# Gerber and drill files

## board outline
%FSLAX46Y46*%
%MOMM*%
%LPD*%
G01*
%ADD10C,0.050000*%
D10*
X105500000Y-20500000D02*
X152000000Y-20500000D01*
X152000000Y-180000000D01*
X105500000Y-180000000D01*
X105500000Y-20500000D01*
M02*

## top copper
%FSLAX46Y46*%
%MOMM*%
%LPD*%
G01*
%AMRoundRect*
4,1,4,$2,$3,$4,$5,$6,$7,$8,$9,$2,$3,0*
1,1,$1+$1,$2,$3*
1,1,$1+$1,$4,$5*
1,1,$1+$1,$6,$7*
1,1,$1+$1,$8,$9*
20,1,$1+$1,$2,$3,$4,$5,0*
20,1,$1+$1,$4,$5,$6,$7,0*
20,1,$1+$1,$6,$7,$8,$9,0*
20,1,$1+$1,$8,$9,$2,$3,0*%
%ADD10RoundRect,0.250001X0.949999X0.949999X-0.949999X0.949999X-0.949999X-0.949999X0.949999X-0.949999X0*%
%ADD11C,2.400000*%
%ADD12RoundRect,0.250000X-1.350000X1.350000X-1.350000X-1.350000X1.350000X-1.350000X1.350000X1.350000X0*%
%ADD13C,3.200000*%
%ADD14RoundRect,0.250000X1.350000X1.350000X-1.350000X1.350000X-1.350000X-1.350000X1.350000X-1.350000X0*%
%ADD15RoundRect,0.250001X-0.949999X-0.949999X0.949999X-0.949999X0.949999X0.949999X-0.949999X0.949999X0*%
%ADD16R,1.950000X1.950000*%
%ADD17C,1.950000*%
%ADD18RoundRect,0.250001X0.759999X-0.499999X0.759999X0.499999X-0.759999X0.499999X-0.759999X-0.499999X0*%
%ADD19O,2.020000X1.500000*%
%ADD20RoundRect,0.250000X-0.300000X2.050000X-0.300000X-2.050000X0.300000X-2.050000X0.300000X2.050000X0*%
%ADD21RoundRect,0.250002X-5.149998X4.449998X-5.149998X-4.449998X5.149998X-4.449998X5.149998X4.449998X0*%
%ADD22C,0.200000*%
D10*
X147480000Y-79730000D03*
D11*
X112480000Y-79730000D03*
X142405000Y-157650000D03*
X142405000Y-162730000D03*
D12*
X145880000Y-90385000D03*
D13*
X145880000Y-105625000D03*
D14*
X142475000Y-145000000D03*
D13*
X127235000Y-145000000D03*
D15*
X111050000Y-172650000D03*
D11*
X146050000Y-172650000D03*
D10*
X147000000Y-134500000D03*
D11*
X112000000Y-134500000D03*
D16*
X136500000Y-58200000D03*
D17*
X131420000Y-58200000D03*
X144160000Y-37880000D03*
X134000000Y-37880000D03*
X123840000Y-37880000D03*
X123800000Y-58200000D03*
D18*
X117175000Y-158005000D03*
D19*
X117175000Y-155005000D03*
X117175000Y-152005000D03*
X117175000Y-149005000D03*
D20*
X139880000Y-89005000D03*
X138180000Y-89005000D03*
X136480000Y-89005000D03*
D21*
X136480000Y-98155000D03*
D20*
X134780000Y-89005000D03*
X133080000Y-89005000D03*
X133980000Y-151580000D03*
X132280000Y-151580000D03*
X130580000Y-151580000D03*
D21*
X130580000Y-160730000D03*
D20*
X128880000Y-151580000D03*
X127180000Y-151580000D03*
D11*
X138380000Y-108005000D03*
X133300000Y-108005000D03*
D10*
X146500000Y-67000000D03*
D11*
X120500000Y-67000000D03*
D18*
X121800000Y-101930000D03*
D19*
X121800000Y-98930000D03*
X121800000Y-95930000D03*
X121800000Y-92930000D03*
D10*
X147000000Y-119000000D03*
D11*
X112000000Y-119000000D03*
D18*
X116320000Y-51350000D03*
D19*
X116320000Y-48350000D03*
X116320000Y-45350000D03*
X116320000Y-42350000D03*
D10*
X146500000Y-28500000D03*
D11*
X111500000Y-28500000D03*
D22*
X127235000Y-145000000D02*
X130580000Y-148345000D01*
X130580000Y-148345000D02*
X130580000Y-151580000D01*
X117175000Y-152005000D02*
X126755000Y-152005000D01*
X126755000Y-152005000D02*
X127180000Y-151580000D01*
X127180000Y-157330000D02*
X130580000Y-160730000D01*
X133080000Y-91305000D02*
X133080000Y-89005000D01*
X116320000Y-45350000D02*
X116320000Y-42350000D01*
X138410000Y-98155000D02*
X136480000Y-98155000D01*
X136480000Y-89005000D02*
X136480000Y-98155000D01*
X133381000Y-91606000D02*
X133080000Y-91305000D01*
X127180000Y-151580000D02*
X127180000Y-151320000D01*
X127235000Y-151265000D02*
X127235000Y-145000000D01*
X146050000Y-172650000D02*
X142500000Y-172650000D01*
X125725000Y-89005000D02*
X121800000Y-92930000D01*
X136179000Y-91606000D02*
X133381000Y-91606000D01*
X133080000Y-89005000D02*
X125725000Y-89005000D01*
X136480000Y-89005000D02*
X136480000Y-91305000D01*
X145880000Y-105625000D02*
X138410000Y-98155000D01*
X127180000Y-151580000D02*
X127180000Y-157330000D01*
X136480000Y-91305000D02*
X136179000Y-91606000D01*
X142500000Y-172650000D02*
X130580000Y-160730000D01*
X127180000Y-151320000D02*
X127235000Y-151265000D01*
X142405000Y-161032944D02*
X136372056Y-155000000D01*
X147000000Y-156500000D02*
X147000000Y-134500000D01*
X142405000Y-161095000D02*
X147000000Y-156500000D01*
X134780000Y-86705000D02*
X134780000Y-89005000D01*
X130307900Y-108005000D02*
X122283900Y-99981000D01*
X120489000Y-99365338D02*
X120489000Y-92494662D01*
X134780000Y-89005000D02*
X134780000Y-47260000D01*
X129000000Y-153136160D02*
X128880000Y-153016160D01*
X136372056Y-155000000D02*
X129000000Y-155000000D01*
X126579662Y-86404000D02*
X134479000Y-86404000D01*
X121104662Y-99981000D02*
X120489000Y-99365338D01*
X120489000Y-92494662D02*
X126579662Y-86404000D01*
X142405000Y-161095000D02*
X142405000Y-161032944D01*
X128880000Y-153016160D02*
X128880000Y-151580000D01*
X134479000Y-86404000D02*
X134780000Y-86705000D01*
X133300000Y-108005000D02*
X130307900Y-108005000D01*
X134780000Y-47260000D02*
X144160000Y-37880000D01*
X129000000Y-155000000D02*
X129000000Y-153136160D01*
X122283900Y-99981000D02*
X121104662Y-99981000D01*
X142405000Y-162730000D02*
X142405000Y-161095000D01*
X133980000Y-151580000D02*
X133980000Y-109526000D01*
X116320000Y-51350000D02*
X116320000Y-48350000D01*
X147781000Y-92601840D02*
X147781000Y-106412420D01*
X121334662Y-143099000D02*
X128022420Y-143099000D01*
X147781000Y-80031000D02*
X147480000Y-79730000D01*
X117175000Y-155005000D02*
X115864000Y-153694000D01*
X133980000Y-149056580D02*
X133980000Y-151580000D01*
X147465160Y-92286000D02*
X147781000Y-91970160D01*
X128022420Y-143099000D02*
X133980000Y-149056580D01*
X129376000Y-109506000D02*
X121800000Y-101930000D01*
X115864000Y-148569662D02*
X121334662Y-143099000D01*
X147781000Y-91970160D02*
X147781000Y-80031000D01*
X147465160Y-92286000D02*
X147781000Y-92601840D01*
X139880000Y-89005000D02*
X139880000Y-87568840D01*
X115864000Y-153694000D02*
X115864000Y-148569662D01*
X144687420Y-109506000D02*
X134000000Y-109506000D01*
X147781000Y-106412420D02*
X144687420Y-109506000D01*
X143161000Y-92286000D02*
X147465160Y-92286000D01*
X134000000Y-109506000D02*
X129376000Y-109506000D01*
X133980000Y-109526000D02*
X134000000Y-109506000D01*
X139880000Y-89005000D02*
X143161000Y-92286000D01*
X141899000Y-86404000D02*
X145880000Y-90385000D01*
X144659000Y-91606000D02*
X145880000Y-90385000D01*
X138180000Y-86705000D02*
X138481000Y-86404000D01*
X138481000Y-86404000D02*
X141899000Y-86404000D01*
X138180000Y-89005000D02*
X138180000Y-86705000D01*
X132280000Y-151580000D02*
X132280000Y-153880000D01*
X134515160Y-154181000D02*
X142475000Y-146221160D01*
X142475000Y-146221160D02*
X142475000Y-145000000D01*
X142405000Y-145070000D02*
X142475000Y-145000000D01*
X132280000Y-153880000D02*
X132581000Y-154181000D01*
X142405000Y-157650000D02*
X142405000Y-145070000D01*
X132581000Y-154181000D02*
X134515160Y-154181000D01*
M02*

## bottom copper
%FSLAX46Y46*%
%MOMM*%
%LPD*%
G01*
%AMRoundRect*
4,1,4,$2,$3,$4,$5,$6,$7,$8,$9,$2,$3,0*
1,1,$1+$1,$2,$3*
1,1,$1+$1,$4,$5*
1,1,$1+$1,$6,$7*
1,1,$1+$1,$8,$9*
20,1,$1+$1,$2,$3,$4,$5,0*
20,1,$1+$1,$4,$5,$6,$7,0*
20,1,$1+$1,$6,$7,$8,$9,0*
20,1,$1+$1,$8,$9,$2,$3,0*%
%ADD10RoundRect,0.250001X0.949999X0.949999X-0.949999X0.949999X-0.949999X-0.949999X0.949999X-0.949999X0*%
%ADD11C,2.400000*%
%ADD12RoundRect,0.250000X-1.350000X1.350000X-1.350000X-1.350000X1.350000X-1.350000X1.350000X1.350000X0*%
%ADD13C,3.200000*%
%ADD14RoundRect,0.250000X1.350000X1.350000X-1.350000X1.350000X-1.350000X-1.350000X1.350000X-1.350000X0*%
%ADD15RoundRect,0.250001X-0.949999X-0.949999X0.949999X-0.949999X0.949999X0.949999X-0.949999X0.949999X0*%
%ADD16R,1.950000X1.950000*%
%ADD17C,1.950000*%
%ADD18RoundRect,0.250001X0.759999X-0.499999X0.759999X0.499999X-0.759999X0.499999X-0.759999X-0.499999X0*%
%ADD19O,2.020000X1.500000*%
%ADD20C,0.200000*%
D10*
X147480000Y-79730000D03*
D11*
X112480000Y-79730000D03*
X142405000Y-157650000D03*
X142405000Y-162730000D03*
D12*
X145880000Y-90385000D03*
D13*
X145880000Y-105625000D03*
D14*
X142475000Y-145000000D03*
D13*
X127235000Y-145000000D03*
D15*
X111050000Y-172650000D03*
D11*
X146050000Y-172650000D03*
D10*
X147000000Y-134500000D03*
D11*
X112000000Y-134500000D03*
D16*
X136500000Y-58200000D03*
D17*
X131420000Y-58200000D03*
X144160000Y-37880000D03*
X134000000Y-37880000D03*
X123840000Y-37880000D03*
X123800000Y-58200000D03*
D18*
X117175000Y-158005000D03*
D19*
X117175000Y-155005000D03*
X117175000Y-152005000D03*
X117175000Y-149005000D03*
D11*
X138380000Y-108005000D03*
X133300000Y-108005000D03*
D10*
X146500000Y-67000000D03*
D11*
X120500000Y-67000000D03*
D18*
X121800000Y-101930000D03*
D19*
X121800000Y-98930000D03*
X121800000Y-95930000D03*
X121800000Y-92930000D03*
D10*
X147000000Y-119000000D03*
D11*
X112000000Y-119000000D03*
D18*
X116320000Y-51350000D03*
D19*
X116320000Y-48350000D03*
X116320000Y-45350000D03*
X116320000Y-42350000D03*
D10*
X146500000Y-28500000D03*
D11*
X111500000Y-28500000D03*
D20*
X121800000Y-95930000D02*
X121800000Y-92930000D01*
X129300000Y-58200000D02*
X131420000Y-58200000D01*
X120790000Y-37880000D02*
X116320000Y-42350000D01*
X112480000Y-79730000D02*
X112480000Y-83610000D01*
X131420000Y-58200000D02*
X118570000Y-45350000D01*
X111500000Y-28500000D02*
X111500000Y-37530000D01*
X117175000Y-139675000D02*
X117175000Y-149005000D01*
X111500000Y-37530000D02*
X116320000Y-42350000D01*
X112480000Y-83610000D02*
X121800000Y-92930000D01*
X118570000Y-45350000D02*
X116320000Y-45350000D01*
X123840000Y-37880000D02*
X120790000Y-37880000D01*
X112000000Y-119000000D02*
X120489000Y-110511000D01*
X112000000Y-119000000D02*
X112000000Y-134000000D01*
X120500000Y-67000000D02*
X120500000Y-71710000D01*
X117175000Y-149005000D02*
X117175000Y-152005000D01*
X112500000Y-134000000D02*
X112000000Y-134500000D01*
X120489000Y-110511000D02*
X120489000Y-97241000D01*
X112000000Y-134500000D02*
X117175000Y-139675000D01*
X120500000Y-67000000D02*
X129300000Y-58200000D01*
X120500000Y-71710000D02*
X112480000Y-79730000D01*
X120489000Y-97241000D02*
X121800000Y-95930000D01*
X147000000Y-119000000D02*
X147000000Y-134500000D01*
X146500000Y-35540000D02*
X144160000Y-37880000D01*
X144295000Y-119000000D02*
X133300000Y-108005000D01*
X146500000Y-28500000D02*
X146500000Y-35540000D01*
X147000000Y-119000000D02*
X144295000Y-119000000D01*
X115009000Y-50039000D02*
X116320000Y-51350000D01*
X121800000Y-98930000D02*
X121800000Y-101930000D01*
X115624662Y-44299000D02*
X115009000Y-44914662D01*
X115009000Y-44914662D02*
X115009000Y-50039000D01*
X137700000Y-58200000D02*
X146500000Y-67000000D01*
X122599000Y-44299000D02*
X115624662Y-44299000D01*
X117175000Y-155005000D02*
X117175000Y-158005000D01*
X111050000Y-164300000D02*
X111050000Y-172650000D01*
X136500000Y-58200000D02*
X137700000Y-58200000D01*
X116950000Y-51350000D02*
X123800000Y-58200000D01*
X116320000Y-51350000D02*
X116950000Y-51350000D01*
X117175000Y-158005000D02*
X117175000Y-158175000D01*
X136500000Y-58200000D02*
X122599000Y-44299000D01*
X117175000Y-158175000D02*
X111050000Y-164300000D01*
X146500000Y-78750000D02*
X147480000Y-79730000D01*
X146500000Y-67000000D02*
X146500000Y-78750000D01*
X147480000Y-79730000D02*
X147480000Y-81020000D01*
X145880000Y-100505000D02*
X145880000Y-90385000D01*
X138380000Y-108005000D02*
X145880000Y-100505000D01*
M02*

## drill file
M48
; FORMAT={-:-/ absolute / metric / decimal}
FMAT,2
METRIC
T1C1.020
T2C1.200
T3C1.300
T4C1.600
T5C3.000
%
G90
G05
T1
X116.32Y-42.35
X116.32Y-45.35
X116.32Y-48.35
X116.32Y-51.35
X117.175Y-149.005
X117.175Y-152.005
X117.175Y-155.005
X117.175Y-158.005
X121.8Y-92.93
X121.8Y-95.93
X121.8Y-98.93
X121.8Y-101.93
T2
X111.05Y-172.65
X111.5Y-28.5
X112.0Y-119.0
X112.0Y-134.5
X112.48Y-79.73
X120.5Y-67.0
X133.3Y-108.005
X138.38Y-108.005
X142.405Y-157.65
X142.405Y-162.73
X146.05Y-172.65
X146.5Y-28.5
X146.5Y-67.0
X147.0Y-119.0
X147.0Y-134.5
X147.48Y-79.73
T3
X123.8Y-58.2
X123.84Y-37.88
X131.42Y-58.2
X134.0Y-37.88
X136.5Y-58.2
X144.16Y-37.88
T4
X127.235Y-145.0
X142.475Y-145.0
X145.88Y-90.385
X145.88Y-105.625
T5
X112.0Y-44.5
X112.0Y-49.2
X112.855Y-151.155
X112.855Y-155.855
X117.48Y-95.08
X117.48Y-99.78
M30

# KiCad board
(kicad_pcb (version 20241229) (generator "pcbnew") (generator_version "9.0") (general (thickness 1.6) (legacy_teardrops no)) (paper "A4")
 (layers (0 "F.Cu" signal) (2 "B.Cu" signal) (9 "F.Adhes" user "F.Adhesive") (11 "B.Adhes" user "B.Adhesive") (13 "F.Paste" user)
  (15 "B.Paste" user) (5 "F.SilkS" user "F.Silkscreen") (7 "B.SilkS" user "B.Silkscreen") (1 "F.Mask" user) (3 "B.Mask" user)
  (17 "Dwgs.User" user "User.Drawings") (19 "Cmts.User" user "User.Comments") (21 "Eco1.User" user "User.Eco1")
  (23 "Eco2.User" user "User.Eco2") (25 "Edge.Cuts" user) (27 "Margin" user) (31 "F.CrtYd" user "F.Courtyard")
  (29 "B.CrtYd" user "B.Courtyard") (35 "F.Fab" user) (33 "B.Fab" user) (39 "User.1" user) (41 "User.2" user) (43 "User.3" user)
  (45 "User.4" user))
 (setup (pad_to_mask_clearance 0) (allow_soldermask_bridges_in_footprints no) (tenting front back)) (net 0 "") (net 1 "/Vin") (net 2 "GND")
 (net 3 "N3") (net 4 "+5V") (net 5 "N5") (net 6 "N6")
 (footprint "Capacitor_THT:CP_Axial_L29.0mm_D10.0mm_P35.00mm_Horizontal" (layer "F.Cu") (at 147.48 79.73 180)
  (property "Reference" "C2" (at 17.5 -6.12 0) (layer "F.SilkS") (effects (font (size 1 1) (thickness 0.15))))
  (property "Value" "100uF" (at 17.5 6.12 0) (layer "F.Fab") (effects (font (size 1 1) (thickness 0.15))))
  (pad "1" thru_hole roundrect (at 0 0 180) (size 2.4 2.4) (drill 1.2) (layers "*.Cu" "*.Mask") (remove_unused_layers no)
   (roundrect_rratio 0.104167) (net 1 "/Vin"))
  (pad "2" thru_hole circle (at 35 0 180) (size 2.4 2.4) (drill 1.2) (layers "*.Cu" "*.Mask") (remove_unused_layers no) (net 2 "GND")))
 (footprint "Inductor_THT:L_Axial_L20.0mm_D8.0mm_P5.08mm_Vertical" (layer "F.Cu") (at 142.405 157.65 -90)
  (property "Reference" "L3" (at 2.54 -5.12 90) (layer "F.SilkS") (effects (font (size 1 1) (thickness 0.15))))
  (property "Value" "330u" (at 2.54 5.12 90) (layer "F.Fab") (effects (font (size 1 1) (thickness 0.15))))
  (pad "1" thru_hole circle (at 0 0 270) (size 2.4 2.4) (drill 1.2) (layers "*.Cu" "*.Mask") (remove_unused_layers no) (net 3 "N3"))
  (pad "2" thru_hole circle (at 5.08 0 270) (size 2.4 2.4) (drill 1.2) (layers "*.Cu" "*.Mask") (remove_unused_layers no) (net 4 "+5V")))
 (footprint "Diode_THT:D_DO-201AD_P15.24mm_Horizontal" (layer "F.Cu") (at 145.88 90.385 -90)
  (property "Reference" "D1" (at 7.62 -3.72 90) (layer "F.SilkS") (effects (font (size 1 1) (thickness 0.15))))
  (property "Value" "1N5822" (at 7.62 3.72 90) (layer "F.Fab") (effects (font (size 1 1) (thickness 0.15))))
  (pad "1" thru_hole roundrect (at 0 0 270) (size 3.2 3.2) (drill 1.6) (layers "*.Cu" "*.Mask") (remove_unused_layers no)
   (roundrect_rratio 0.078125) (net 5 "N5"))
  (pad "2" thru_hole circle (at 15.24 0 270) (size 3.2 3.2) (drill 1.6) (layers "*.Cu" "*.Mask") (remove_unused_layers no) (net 2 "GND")))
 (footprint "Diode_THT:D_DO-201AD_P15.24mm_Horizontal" (layer "F.Cu") (at 142.475 145 180)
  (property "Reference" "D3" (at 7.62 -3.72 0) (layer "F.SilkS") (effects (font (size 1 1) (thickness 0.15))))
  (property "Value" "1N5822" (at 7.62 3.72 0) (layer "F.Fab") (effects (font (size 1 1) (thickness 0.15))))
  (pad "1" thru_hole roundrect (at 0 0 180) (size 3.2 3.2) (drill 1.6) (layers "*.Cu" "*.Mask") (remove_unused_layers no)
   (roundrect_rratio 0.078125) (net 3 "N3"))
  (pad "2" thru_hole circle (at 15.24 0 180) (size 3.2 3.2) (drill 1.6) (layers "*.Cu" "*.Mask") (remove_unused_layers no) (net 2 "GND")))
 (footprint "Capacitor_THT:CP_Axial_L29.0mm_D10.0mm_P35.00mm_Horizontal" (layer "F.Cu") (at 111.05 172.65)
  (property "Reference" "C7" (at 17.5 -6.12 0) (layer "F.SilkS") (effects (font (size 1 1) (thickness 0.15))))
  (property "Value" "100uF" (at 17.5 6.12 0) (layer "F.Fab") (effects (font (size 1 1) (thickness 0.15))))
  (pad "1" thru_hole roundrect (at 0 0) (size 2.4 2.4) (drill 1.2) (layers "*.Cu" "*.Mask") (remove_unused_layers no)
   (roundrect_rratio 0.104167) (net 1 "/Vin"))
  (pad "2" thru_hole circle (at 35 0) (size 2.4 2.4) (drill 1.2) (layers "*.Cu" "*.Mask") (remove_unused_layers no) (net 2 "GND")))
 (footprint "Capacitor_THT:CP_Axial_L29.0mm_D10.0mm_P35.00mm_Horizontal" (layer "F.Cu") (at 147 134.5 180)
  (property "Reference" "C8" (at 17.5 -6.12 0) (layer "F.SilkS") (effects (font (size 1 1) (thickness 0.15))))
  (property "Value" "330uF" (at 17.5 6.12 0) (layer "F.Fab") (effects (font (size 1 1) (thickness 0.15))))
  (pad "1" thru_hole roundrect (at 0 0 180) (size 2.4 2.4) (drill 1.2) (layers "*.Cu" "*.Mask") (remove_unused_layers no)
   (roundrect_rratio 0.104167) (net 4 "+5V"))
  (pad "2" thru_hole circle (at 35 0 180) (size 2.4 2.4) (drill 1.2) (layers "*.Cu" "*.Mask") (remove_unused_layers no) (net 2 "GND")))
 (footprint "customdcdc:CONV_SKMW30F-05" (layer "F.Cu") (at 134 48 180)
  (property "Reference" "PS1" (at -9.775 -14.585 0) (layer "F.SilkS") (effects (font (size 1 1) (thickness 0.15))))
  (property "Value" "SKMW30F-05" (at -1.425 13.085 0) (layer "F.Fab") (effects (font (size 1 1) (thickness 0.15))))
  (pad "1" thru_hole rect (at -2.5 -10.2 180) (size 1.95 1.95) (drill 1.3) (layers "*.Cu" "*.Mask") (remove_unused_layers no) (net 1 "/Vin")
   (solder_mask_margin 0.102))
  (pad "2" thru_hole circle (at 2.58 -10.2 180) (size 1.95 1.95) (drill 1.3) (layers "*.Cu" "*.Mask") (remove_unused_layers no)
   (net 2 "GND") (solder_mask_margin 0.102))
  (pad "3" thru_hole circle (at -10.16 10.12 180) (size 1.95 1.95) (drill 1.3) (layers "*.Cu" "*.Mask") (remove_unused_layers no)
   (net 4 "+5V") (solder_mask_margin 0.102))
  (pad "4" thru_hole circle (at 0 10.12 180) (size 1.95 1.95) (drill 1.3) (layers "*.Cu" "*.Mask") (remove_unused_layers no) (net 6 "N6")
   (solder_mask_margin 0.102))
  (pad "5" thru_hole circle (at 10.16 10.12 180) (size 1.95 1.95) (drill 1.3) (layers "*.Cu" "*.Mask") (remove_unused_layers no)
   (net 2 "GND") (solder_mask_margin 0.102))
  (pad "6" thru_hole circle (at 10.2 -10.2 180) (size 1.95 1.95) (drill 1.3) (layers "*.Cu" "*.Mask") (remove_unused_layers no)
   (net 1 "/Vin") (solder_mask_margin 0.102)))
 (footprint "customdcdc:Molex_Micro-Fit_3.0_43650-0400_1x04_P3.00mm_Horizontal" (layer "F.Cu") (at 117.175 158.005 90)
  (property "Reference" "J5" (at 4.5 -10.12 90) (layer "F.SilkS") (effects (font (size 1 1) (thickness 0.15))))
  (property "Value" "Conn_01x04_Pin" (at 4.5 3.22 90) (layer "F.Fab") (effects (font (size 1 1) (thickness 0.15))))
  (pad "" np_thru_hole circle (at 2.15 -4.32 90) (size 3 3) (drill 3) (layers "*.Cu" "*.Mask"))
  (pad "" np_thru_hole circle (at 6.85 -4.32 90) (size 3 3) (drill 3) (layers "*.Cu" "*.Mask"))
  (pad "1" thru_hole roundrect (at 0 0 90) (size 1.5 2.02) (drill 1.02) (layers "*.Cu" "*.Mask") (remove_unused_layers no)
   (roundrect_rratio 0.166667) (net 1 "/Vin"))
  (pad "2" thru_hole oval (at 3 0 90) (size 1.5 2.02) (drill 1.02) (layers "*.Cu" "*.Mask") (remove_unused_layers no) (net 1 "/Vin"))
  (pad "3" thru_hole oval (at 6 0 90) (size 1.5 2.02) (drill 1.02) (layers "*.Cu" "*.Mask") (remove_unused_layers no) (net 2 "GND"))
  (pad "4" thru_hole oval (at 9 0 90) (size 1.5 2.02) (drill 1.02) (layers "*.Cu" "*.Mask") (remove_unused_layers no) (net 2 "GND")))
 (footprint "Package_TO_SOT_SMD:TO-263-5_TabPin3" (layer "F.Cu") (at 136.48 96.655 -90)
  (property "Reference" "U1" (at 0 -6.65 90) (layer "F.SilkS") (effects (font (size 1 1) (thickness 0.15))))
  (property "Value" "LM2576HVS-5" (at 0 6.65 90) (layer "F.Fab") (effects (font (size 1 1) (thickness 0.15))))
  (pad "" smd roundrect (at -0.925 -2.775 270) (size 4.55 5.25) (layers "F.Paste") (roundrect_rratio 0.054945))
  (pad "" smd roundrect (at -0.925 2.775 270) (size 4.55 5.25) (layers "F.Paste") (roundrect_rratio 0.054945))
  (pad "" smd roundrect (at 3.925 -2.775 270) (size 4.55 5.25) (layers "F.Paste") (roundrect_rratio 0.054945))
  (pad "" smd roundrect (at 3.925 2.775 270) (size 4.55 5.25) (layers "F.Paste") (roundrect_rratio 0.054945))
  (pad "1" smd roundrect (at -7.65 -3.4 270) (size 4.6 1.1) (layers "F.Cu" "F.Mask" "F.Paste") (roundrect_rratio 0.227273) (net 1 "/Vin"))
  (pad "2" smd roundrect (at -7.65 -1.7 270) (size 4.6 1.1) (layers "F.Cu" "F.Mask" "F.Paste") (roundrect_rratio 0.227273) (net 5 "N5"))
  (pad "3" smd roundrect (at -7.65 0 270) (size 4.6 1.1) (layers "F.Cu" "F.Mask" "F.Paste") (roundrect_rratio 0.227273) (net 2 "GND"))
  (pad "3" smd roundrect (at 1.5 0 270) (size 9.4 10.8) (layers "F.Cu" "F.Mask") (roundrect_rratio 0.026596) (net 2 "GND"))
  (pad "4" smd roundrect (at -7.65 1.7 270) (size 4.6 1.1) (layers "F.Cu" "F.Mask" "F.Paste") (roundrect_rratio 0.227273) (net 4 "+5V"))
  (pad "5" smd roundrect (at -7.65 3.4 270) (size 4.6 1.1) (layers "F.Cu" "F.Mask" "F.Paste") (roundrect_rratio 0.227273) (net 2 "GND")))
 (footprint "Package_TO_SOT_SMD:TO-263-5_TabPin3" (layer "F.Cu") (at 130.58 159.23 -90)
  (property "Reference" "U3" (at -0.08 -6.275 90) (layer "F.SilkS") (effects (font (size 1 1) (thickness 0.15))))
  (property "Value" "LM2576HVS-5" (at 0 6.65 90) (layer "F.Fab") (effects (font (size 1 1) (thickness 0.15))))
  (pad "" smd roundrect (at -0.925 -2.775 270) (size 4.55 5.25) (layers "F.Paste") (roundrect_rratio 0.054945))
  (pad "" smd roundrect (at -0.925 2.775 270) (size 4.55 5.25) (layers "F.Paste") (roundrect_rratio 0.054945))
  (pad "" smd roundrect (at 3.925 -2.775 270) (size 4.55 5.25) (layers "F.Paste") (roundrect_rratio 0.054945))
  (pad "" smd roundrect (at 3.925 2.775 270) (size 4.55 5.25) (layers "F.Paste") (roundrect_rratio 0.054945))
  (pad "1" smd roundrect (at -7.65 -3.4 270) (size 4.6 1.1) (layers "F.Cu" "F.Mask" "F.Paste") (roundrect_rratio 0.227273) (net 1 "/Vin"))
  (pad "2" smd roundrect (at -7.65 -1.7 270) (size 4.6 1.1) (layers "F.Cu" "F.Mask" "F.Paste") (roundrect_rratio 0.227273) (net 3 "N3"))
  (pad "3" smd roundrect (at -7.65 0 270) (size 4.6 1.1) (layers "F.Cu" "F.Mask" "F.Paste") (roundrect_rratio 0.227273) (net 2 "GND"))
  (pad "3" smd roundrect (at 1.5 0 270) (size 9.4 10.8) (layers "F.Cu" "F.Mask") (roundrect_rratio 0.026596) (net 2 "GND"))
  (pad "4" smd roundrect (at -7.65 1.7 270) (size 4.6 1.1) (layers "F.Cu" "F.Mask" "F.Paste") (roundrect_rratio 0.227273) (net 4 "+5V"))
  (pad "5" smd roundrect (at -7.65 3.4 270) (size 4.6 1.1) (layers "F.Cu" "F.Mask" "F.Paste") (roundrect_rratio 0.227273) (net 2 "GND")))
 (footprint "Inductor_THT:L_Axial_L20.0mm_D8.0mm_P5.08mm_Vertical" (layer "F.Cu") (at 138.38 108.005 180)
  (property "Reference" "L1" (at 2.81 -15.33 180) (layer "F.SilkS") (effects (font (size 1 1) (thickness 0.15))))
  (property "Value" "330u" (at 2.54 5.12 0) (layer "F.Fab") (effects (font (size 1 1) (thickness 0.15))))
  (pad "1" thru_hole circle (at 0 0 180) (size 2.4 2.4) (drill 1.2) (layers "*.Cu" "*.Mask") (remove_unused_layers no) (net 5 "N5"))
  (pad "2" thru_hole circle (at 5.08 0 180) (size 2.4 2.4) (drill 1.2) (layers "*.Cu" "*.Mask") (remove_unused_layers no) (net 4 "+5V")))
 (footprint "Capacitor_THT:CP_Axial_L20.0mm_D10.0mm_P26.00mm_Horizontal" (layer "F.Cu") (at 146.5 67 180)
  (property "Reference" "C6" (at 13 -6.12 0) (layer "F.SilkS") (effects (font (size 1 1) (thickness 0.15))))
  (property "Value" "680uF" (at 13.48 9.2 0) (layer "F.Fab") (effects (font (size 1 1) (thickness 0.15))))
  (pad "1" thru_hole roundrect (at 0 0 180) (size 2.4 2.4) (drill 1.2) (layers "*.Cu" "*.Mask") (remove_unused_layers no)
   (roundrect_rratio 0.104167) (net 1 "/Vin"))
  (pad "2" thru_hole circle (at 26 0 180) (size 2.4 2.4) (drill 1.2) (layers "*.Cu" "*.Mask") (remove_unused_layers no) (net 2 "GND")))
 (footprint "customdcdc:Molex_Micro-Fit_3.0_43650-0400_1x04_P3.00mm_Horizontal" (layer "F.Cu") (at 121.8 101.93 90)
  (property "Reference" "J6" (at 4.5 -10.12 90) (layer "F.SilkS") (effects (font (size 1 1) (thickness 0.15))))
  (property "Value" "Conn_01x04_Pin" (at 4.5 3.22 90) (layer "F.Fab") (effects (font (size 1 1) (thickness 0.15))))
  (pad "" np_thru_hole circle (at 2.15 -4.32 90) (size 3 3) (drill 3) (layers "*.Cu" "*.Mask"))
  (pad "" np_thru_hole circle (at 6.85 -4.32 90) (size 3 3) (drill 3) (layers "*.Cu" "*.Mask"))
  (pad "1" thru_hole roundrect (at 0 0 90) (size 1.5 2.02) (drill 1.02) (layers "*.Cu" "*.Mask") (remove_unused_layers no)
   (roundrect_rratio 0.166667) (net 1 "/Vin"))
  (pad "2" thru_hole oval (at 3 0 90) (size 1.5 2.02) (drill 1.02) (layers "*.Cu" "*.Mask") (remove_unused_layers no) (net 1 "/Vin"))
  (pad "3" thru_hole oval (at 6 0 90) (size 1.5 2.02) (drill 1.02) (layers "*.Cu" "*.Mask") (remove_unused_layers no) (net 2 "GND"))
  (pad "4" thru_hole oval (at 9 0 90) (size 1.5 2.02) (drill 1.02) (layers "*.Cu" "*.Mask") (remove_unused_layers no) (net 2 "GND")))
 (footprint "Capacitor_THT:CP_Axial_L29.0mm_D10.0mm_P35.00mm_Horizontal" (layer "F.Cu") (at 147 119 180)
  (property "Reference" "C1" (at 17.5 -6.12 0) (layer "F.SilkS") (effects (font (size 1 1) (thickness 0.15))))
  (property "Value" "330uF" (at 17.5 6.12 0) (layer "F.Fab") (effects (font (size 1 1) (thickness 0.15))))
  (pad "1" thru_hole roundrect (at 0 0 180) (size 2.4 2.4) (drill 1.2) (layers "*.Cu" "*.Mask") (remove_unused_layers no)
   (roundrect_rratio 0.104167) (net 4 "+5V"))
  (pad "2" thru_hole circle (at 35 0 180) (size 2.4 2.4) (drill 1.2) (layers "*.Cu" "*.Mask") (remove_unused_layers no) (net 2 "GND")))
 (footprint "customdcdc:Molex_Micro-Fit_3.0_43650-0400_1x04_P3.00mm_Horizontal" (layer "F.Cu") (at 116.32 51.35 90)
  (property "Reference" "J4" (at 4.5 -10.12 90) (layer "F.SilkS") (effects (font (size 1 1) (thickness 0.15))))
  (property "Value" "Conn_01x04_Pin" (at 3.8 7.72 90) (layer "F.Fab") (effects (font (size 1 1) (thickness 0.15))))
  (pad "" np_thru_hole circle (at 2.15 -4.32 90) (size 3 3) (drill 3) (layers "*.Cu" "*.Mask"))
  (pad "" np_thru_hole circle (at 6.85 -4.32 90) (size 3 3) (drill 3) (layers "*.Cu" "*.Mask"))
  (pad "1" thru_hole roundrect (at 0 0 90) (size 1.5 2.02) (drill 1.02) (layers "*.Cu" "*.Mask") (remove_unused_layers no)
   (roundrect_rratio 0.166667) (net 1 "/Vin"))
  (pad "2" thru_hole oval (at 3 0 90) (size 1.5 2.02) (drill 1.02) (layers "*.Cu" "*.Mask") (remove_unused_layers no) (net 1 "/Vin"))
  (pad "3" thru_hole oval (at 6 0 90) (size 1.5 2.02) (drill 1.02) (layers "*.Cu" "*.Mask") (remove_unused_layers no) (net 2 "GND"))
  (pad "4" thru_hole oval (at 9 0 90) (size 1.5 2.02) (drill 1.02) (layers "*.Cu" "*.Mask") (remove_unused_layers no) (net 2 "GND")))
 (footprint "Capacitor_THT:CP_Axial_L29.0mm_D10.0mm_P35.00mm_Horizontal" (layer "F.Cu") (at 146.5 28.5 180)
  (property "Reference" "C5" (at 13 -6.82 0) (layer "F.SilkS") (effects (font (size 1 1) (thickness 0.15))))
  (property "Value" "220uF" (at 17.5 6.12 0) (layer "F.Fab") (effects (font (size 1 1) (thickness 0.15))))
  (pad "1" thru_hole roundrect (at 0 0 180) (size 2.4 2.4) (drill 1.2) (layers "*.Cu" "*.Mask") (remove_unused_layers no)
   (roundrect_rratio 0.104167) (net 4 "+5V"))
  (pad "2" thru_hole circle (at 35 0 180) (size 2.4 2.4) (drill 1.2) (layers "*.Cu" "*.Mask") (remove_unused_layers no) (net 2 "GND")))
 (gr_rect (start 105.5 20.5) (end 152 180) (stroke (width 0.05) (type default)) (fill no) (layer "Edge.Cuts"))
 (segment (start 127.235 145) (end 130.58 148.345) (width 0.2) (layer "F.Cu") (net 2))
 (segment (start 130.58 148.345) (end 130.58 151.58) (width 0.2) (layer "F.Cu") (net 2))
 (segment (start 117.175 152.005) (end 126.755 152.005) (width 0.2) (layer "F.Cu") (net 2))
 (segment (start 126.755 152.005) (end 127.18 151.58) (width 0.2) (layer "F.Cu") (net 2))
 (segment (start 127.18 157.33) (end 130.58 160.73) (width 0.2) (layer "F.Cu") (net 2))
 (segment (start 133.08 91.305) (end 133.08 89.005) (width 0.2) (layer "F.Cu") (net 2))
 (segment (start 116.32 45.35) (end 116.32 42.35) (width 0.2) (layer "F.Cu") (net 2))
 (segment (start 138.41 98.155) (end 136.48 98.155) (width 0.2) (layer "F.Cu") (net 2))
 (segment (start 136.48 89.005) (end 136.48 98.155) (width 0.2) (layer "F.Cu") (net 2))
 (segment (start 133.381 91.606) (end 133.08 91.305) (width 0.2) (layer "F.Cu") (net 2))
 (segment (start 127.18 151.58) (end 127.18 151.32) (width 0.2) (layer "F.Cu") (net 2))
 (segment (start 127.235 151.265) (end 127.235 145) (width 0.2) (layer "F.Cu") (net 2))
 (segment (start 146.05 172.65) (end 142.5 172.65) (width 0.2) (layer "F.Cu") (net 2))
 (segment (start 125.725 89.005) (end 121.8 92.93) (width 0.2) (layer "F.Cu") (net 2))
 (segment (start 136.179 91.606) (end 133.381 91.606) (width 0.2) (layer "F.Cu") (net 2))
 (segment (start 133.08 89.005) (end 125.725 89.005) (width 0.2) (layer "F.Cu") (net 2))
 (segment (start 136.48 89.005) (end 136.48 91.305) (width 0.2) (layer "F.Cu") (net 2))
 (segment (start 145.88 105.625) (end 138.41 98.155) (width 0.2) (layer "F.Cu") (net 2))
 (segment (start 127.18 151.58) (end 127.18 157.33) (width 0.2) (layer "F.Cu") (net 2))
 (segment (start 136.48 91.305) (end 136.179 91.606) (width 0.2) (layer "F.Cu") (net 2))
 (segment (start 142.5 172.65) (end 130.58 160.73) (width 0.2) (layer "F.Cu") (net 2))
 (segment (start 127.18 151.32) (end 127.235 151.265) (width 0.2) (layer "F.Cu") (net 2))
 (segment (start 121.8 95.93) (end 121.8 92.93) (width 0.2) (layer "B.Cu") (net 2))
 (segment (start 129.3 58.2) (end 131.42 58.2) (width 0.2) (layer "B.Cu") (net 2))
 (segment (start 120.79 37.88) (end 116.32 42.35) (width 0.2) (layer "B.Cu") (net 2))
 (segment (start 112.48 79.73) (end 112.48 83.61) (width 0.2) (layer "B.Cu") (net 2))
 (segment (start 131.42 58.2) (end 118.57 45.35) (width 0.2) (layer "B.Cu") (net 2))
 (segment (start 111.5 28.5) (end 111.5 37.53) (width 0.2) (layer "B.Cu") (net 2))
 (segment (start 117.175 139.675) (end 117.175 149.005) (width 0.2) (layer "B.Cu") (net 2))
 (segment (start 111.5 37.53) (end 116.32 42.35) (width 0.2) (layer "B.Cu") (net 2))
 (segment (start 112.48 83.61) (end 121.8 92.93) (width 0.2) (layer "B.Cu") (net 2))
 (segment (start 118.57 45.35) (end 116.32 45.35) (width 0.2) (layer "B.Cu") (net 2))
 (segment (start 123.84 37.88) (end 120.79 37.88) (width 0.2) (layer "B.Cu") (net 2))
 (segment (start 112 119) (end 120.489 110.511) (width 0.2) (layer "B.Cu") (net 2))
 (segment (start 112 119) (end 112 134) (width 0.2) (layer "B.Cu") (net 2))
 (segment (start 120.5 67) (end 120.5 71.71) (width 0.2) (layer "B.Cu") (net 2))
 (segment (start 117.175 149.005) (end 117.175 152.005) (width 0.2) (layer "B.Cu") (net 2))
 (segment (start 112.5 134) (end 112 134.5) (width 0.2) (layer "B.Cu") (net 2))
 (segment (start 120.489 110.511) (end 120.489 97.241) (width 0.2) (layer "B.Cu") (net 2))
 (segment (start 112 134.5) (end 117.175 139.675) (width 0.2) (layer "B.Cu") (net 2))
 (segment (start 120.5 67) (end 129.3 58.2) (width 0.2) (layer "B.Cu") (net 2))
 (segment (start 120.5 71.71) (end 112.48 79.73) (width 0.2) (layer "B.Cu") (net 2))
 (segment (start 120.489 97.241) (end 121.8 95.93) (width 0.2) (layer "B.Cu") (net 2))
 (segment (start 142.405 161.032944) (end 136.372056 155) (width 0.2) (layer "F.Cu") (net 4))
 (segment (start 147 156.5) (end 147 134.5) (width 0.2) (layer "F.Cu") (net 4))
 (segment (start 142.405 161.095) (end 147 156.5) (width 0.2) (layer "F.Cu") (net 4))
 (segment (start 134.78 86.705) (end 134.78 89.005) (width 0.2) (layer "F.Cu") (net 4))
 (segment (start 130.3079 108.005) (end 122.2839 99.981) (width 0.2) (layer "F.Cu") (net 4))
 (segment (start 120.489 99.365338) (end 120.489 92.494662) (width 0.2) (layer "F.Cu") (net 4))
 (segment (start 134.78 89.005) (end 134.78 47.26) (width 0.2) (layer "F.Cu") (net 4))
 (segment (start 129 153.13616) (end 128.88 153.01616) (width 0.2) (layer "F.Cu") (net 4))
 (segment (start 136.372056 155) (end 129 155) (width 0.2) (layer "F.Cu") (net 4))
 (segment (start 126.579662 86.404) (end 134.479 86.404) (width 0.2) (layer "F.Cu") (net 4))
 (segment (start 121.104662 99.981) (end 120.489 99.365338) (width 0.2) (layer "F.Cu") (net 4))
 (segment (start 120.489 92.494662) (end 126.579662 86.404) (width 0.2) (layer "F.Cu") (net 4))
 (segment (start 142.405 161.095) (end 142.405 161.032944) (width 0.2) (layer "F.Cu") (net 4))
 (segment (start 128.88 153.01616) (end 128.88 151.58) (width 0.2) (layer "F.Cu") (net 4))
 (segment (start 134.479 86.404) (end 134.78 86.705) (width 0.2) (layer "F.Cu") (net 4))
 (segment (start 133.3 108.005) (end 130.3079 108.005) (width 0.2) (layer "F.Cu") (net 4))
 (segment (start 134.78 47.26) (end 144.16 37.88) (width 0.2) (layer "F.Cu") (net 4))
 (segment (start 129 155) (end 129 153.13616) (width 0.2) (layer "F.Cu") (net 4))
 (segment (start 122.2839 99.981) (end 121.104662 99.981) (width 0.2) (layer "F.Cu") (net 4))
 (segment (start 142.405 162.73) (end 142.405 161.095) (width 0.2) (layer "F.Cu") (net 4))
 (segment (start 147 119) (end 147 134.5) (width 0.2) (layer "B.Cu") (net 4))
 (segment (start 146.5 35.54) (end 144.16 37.88) (width 0.2) (layer "B.Cu") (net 4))
 (segment (start 144.295 119) (end 133.3 108.005) (width 0.2) (layer "B.Cu") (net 4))
 (segment (start 146.5 28.5) (end 146.5 35.54) (width 0.2) (layer "B.Cu") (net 4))
 (segment (start 147 119) (end 144.295 119) (width 0.2) (layer "B.Cu") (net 4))
 (segment (start 133.98 151.58) (end 133.98 109.526) (width 0.2) (layer "F.Cu") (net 1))
 (segment (start 116.32 51.35) (end 116.32 48.35) (width 0.2) (layer "F.Cu") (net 1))
 (segment (start 147.781 92.60184) (end 147.781 106.41242) (width 0.2) (layer "F.Cu") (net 1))
 (segment (start 121.334662 143.099) (end 128.02242 143.099) (width 0.2) (layer "F.Cu") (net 1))
 (segment (start 147.781 80.031) (end 147.48 79.73) (width 0.2) (layer "F.Cu") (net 1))
 (segment (start 117.175 155.005) (end 115.864 153.694) (width 0.2) (layer "F.Cu") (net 1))
 (segment (start 133.98 149.05658) (end 133.98 151.58) (width 0.2) (layer "F.Cu") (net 1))
 (segment (start 147.46516 92.286) (end 147.781 91.97016) (width 0.2) (layer "F.Cu") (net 1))
 (segment (start 128.02242 143.099) (end 133.98 149.05658) (width 0.2) (layer "F.Cu") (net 1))
 (segment (start 129.376 109.506) (end 121.8 101.93) (width 0.2) (layer "F.Cu") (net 1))
 (segment (start 115.864 148.569662) (end 121.334662 143.099) (width 0.2) (layer "F.Cu") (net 1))
 (segment (start 147.781 91.97016) (end 147.781 80.031) (width 0.2) (layer "F.Cu") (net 1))
 (segment (start 147.46516 92.286) (end 147.781 92.60184) (width 0.2) (layer "F.Cu") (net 1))
 (segment (start 139.88 89.005) (end 139.88 87.56884) (width 0.2) (layer "F.Cu") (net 1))
 (segment (start 115.864 153.694) (end 115.864 148.569662) (width 0.2) (layer "F.Cu") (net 1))
 (segment (start 144.68742 109.506) (end 134 109.506) (width 0.2) (layer "F.Cu") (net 1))
 (segment (start 147.781 106.41242) (end 144.68742 109.506) (width 0.2) (layer "F.Cu") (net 1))
 (segment (start 143.161 92.286) (end 147.46516 92.286) (width 0.2) (layer "F.Cu") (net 1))
 (segment (start 134 109.506) (end 129.376 109.506) (width 0.2) (layer "F.Cu") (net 1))
 (segment (start 133.98 109.526) (end 134 109.506) (width 0.2) (layer "F.Cu") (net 1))
 (segment (start 139.88 89.005) (end 143.161 92.286) (width 0.2) (layer "F.Cu") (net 1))
 (segment (start 115.009 50.039) (end 116.32 51.35) (width 0.2) (layer "B.Cu") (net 1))
 (segment (start 121.8 98.93) (end 121.8 101.93) (width 0.2) (layer "B.Cu") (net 1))
 (segment (start 115.624662 44.299) (end 115.009 44.914662) (width 0.2) (layer "B.Cu") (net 1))
 (segment (start 115.009 44.914662) (end 115.009 50.039) (width 0.2) (layer "B.Cu") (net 1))
 (segment (start 137.7 58.2) (end 146.5 67) (width 0.2) (layer "B.Cu") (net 1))
 (segment (start 122.599 44.299) (end 115.624662 44.299) (width 0.2) (layer "B.Cu") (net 1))
 (segment (start 117.175 155.005) (end 117.175 158.005) (width 0.2) (layer "B.Cu") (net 1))
 (segment (start 111.05 164.3) (end 111.05 172.65) (width 0.2) (layer "B.Cu") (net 1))
 (segment (start 136.5 58.2) (end 137.7 58.2) (width 0.2) (layer "B.Cu") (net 1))
 (segment (start 116.95 51.35) (end 123.8 58.2) (width 0.2) (layer "B.Cu") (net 1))
 (segment (start 116.32 51.35) (end 116.95 51.35) (width 0.2) (layer "B.Cu") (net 1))
 (segment (start 117.175 158.005) (end 117.175 158.175) (width 0.2) (layer "B.Cu") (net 1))
 (segment (start 136.5 58.2) (end 122.599 44.299) (width 0.2) (layer "B.Cu") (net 1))
 (segment (start 117.175 158.175) (end 111.05 164.3) (width 0.2) (layer "B.Cu") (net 1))
 (segment (start 146.5 78.75) (end 147.48 79.73) (width 0.2) (layer "B.Cu") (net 1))
 (segment (start 146.5 67) (end 146.5 78.75) (width 0.2) (layer "B.Cu") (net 1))
 (segment (start 147.48 79.73) (end 147.48 81.02) (width 0.2) (layer "B.Cu") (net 1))
 (segment (start 141.899 86.404) (end 145.88 90.385) (width 0.2) (layer "F.Cu") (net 5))
 (segment (start 144.659 91.606) (end 145.88 90.385) (width 0.2) (layer "F.Cu") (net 5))
 (segment (start 138.18 86.705) (end 138.481 86.404) (width 0.2) (layer "F.Cu") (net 5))
 (segment (start 138.481 86.404) (end 141.899 86.404) (width 0.2) (layer "F.Cu") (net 5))
 (segment (start 138.18 89.005) (end 138.18 86.705) (width 0.2) (layer "F.Cu") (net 5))
 (segment (start 145.88 100.505) (end 145.88 90.385) (width 0.2) (layer "B.Cu") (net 5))
 (segment (start 138.38 108.005) (end 145.88 100.505) (width 0.2) (layer "B.Cu") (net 5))
 (segment (start 132.28 151.58) (end 132.28 153.88) (width 0.2) (layer "F.Cu") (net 3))
 (segment (start 134.51516 154.181) (end 142.475 146.22116) (width 0.2) (layer "F.Cu") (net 3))
 (segment (start 142.475 146.22116) (end 142.475 145) (width 0.2) (layer "F.Cu") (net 3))
 (segment (start 142.405 145.07) (end 142.475 145) (width 0.2) (layer "F.Cu") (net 3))
 (segment (start 132.28 153.88) (end 132.581 154.181) (width 0.2) (layer "F.Cu") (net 3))
 (segment (start 142.405 157.65) (end 142.405 145.07) (width 0.2) (layer "F.Cu") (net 3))
 (segment (start 132.581 154.181) (end 134.51516 154.181) (width 0.2) (layer "F.Cu") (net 3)))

